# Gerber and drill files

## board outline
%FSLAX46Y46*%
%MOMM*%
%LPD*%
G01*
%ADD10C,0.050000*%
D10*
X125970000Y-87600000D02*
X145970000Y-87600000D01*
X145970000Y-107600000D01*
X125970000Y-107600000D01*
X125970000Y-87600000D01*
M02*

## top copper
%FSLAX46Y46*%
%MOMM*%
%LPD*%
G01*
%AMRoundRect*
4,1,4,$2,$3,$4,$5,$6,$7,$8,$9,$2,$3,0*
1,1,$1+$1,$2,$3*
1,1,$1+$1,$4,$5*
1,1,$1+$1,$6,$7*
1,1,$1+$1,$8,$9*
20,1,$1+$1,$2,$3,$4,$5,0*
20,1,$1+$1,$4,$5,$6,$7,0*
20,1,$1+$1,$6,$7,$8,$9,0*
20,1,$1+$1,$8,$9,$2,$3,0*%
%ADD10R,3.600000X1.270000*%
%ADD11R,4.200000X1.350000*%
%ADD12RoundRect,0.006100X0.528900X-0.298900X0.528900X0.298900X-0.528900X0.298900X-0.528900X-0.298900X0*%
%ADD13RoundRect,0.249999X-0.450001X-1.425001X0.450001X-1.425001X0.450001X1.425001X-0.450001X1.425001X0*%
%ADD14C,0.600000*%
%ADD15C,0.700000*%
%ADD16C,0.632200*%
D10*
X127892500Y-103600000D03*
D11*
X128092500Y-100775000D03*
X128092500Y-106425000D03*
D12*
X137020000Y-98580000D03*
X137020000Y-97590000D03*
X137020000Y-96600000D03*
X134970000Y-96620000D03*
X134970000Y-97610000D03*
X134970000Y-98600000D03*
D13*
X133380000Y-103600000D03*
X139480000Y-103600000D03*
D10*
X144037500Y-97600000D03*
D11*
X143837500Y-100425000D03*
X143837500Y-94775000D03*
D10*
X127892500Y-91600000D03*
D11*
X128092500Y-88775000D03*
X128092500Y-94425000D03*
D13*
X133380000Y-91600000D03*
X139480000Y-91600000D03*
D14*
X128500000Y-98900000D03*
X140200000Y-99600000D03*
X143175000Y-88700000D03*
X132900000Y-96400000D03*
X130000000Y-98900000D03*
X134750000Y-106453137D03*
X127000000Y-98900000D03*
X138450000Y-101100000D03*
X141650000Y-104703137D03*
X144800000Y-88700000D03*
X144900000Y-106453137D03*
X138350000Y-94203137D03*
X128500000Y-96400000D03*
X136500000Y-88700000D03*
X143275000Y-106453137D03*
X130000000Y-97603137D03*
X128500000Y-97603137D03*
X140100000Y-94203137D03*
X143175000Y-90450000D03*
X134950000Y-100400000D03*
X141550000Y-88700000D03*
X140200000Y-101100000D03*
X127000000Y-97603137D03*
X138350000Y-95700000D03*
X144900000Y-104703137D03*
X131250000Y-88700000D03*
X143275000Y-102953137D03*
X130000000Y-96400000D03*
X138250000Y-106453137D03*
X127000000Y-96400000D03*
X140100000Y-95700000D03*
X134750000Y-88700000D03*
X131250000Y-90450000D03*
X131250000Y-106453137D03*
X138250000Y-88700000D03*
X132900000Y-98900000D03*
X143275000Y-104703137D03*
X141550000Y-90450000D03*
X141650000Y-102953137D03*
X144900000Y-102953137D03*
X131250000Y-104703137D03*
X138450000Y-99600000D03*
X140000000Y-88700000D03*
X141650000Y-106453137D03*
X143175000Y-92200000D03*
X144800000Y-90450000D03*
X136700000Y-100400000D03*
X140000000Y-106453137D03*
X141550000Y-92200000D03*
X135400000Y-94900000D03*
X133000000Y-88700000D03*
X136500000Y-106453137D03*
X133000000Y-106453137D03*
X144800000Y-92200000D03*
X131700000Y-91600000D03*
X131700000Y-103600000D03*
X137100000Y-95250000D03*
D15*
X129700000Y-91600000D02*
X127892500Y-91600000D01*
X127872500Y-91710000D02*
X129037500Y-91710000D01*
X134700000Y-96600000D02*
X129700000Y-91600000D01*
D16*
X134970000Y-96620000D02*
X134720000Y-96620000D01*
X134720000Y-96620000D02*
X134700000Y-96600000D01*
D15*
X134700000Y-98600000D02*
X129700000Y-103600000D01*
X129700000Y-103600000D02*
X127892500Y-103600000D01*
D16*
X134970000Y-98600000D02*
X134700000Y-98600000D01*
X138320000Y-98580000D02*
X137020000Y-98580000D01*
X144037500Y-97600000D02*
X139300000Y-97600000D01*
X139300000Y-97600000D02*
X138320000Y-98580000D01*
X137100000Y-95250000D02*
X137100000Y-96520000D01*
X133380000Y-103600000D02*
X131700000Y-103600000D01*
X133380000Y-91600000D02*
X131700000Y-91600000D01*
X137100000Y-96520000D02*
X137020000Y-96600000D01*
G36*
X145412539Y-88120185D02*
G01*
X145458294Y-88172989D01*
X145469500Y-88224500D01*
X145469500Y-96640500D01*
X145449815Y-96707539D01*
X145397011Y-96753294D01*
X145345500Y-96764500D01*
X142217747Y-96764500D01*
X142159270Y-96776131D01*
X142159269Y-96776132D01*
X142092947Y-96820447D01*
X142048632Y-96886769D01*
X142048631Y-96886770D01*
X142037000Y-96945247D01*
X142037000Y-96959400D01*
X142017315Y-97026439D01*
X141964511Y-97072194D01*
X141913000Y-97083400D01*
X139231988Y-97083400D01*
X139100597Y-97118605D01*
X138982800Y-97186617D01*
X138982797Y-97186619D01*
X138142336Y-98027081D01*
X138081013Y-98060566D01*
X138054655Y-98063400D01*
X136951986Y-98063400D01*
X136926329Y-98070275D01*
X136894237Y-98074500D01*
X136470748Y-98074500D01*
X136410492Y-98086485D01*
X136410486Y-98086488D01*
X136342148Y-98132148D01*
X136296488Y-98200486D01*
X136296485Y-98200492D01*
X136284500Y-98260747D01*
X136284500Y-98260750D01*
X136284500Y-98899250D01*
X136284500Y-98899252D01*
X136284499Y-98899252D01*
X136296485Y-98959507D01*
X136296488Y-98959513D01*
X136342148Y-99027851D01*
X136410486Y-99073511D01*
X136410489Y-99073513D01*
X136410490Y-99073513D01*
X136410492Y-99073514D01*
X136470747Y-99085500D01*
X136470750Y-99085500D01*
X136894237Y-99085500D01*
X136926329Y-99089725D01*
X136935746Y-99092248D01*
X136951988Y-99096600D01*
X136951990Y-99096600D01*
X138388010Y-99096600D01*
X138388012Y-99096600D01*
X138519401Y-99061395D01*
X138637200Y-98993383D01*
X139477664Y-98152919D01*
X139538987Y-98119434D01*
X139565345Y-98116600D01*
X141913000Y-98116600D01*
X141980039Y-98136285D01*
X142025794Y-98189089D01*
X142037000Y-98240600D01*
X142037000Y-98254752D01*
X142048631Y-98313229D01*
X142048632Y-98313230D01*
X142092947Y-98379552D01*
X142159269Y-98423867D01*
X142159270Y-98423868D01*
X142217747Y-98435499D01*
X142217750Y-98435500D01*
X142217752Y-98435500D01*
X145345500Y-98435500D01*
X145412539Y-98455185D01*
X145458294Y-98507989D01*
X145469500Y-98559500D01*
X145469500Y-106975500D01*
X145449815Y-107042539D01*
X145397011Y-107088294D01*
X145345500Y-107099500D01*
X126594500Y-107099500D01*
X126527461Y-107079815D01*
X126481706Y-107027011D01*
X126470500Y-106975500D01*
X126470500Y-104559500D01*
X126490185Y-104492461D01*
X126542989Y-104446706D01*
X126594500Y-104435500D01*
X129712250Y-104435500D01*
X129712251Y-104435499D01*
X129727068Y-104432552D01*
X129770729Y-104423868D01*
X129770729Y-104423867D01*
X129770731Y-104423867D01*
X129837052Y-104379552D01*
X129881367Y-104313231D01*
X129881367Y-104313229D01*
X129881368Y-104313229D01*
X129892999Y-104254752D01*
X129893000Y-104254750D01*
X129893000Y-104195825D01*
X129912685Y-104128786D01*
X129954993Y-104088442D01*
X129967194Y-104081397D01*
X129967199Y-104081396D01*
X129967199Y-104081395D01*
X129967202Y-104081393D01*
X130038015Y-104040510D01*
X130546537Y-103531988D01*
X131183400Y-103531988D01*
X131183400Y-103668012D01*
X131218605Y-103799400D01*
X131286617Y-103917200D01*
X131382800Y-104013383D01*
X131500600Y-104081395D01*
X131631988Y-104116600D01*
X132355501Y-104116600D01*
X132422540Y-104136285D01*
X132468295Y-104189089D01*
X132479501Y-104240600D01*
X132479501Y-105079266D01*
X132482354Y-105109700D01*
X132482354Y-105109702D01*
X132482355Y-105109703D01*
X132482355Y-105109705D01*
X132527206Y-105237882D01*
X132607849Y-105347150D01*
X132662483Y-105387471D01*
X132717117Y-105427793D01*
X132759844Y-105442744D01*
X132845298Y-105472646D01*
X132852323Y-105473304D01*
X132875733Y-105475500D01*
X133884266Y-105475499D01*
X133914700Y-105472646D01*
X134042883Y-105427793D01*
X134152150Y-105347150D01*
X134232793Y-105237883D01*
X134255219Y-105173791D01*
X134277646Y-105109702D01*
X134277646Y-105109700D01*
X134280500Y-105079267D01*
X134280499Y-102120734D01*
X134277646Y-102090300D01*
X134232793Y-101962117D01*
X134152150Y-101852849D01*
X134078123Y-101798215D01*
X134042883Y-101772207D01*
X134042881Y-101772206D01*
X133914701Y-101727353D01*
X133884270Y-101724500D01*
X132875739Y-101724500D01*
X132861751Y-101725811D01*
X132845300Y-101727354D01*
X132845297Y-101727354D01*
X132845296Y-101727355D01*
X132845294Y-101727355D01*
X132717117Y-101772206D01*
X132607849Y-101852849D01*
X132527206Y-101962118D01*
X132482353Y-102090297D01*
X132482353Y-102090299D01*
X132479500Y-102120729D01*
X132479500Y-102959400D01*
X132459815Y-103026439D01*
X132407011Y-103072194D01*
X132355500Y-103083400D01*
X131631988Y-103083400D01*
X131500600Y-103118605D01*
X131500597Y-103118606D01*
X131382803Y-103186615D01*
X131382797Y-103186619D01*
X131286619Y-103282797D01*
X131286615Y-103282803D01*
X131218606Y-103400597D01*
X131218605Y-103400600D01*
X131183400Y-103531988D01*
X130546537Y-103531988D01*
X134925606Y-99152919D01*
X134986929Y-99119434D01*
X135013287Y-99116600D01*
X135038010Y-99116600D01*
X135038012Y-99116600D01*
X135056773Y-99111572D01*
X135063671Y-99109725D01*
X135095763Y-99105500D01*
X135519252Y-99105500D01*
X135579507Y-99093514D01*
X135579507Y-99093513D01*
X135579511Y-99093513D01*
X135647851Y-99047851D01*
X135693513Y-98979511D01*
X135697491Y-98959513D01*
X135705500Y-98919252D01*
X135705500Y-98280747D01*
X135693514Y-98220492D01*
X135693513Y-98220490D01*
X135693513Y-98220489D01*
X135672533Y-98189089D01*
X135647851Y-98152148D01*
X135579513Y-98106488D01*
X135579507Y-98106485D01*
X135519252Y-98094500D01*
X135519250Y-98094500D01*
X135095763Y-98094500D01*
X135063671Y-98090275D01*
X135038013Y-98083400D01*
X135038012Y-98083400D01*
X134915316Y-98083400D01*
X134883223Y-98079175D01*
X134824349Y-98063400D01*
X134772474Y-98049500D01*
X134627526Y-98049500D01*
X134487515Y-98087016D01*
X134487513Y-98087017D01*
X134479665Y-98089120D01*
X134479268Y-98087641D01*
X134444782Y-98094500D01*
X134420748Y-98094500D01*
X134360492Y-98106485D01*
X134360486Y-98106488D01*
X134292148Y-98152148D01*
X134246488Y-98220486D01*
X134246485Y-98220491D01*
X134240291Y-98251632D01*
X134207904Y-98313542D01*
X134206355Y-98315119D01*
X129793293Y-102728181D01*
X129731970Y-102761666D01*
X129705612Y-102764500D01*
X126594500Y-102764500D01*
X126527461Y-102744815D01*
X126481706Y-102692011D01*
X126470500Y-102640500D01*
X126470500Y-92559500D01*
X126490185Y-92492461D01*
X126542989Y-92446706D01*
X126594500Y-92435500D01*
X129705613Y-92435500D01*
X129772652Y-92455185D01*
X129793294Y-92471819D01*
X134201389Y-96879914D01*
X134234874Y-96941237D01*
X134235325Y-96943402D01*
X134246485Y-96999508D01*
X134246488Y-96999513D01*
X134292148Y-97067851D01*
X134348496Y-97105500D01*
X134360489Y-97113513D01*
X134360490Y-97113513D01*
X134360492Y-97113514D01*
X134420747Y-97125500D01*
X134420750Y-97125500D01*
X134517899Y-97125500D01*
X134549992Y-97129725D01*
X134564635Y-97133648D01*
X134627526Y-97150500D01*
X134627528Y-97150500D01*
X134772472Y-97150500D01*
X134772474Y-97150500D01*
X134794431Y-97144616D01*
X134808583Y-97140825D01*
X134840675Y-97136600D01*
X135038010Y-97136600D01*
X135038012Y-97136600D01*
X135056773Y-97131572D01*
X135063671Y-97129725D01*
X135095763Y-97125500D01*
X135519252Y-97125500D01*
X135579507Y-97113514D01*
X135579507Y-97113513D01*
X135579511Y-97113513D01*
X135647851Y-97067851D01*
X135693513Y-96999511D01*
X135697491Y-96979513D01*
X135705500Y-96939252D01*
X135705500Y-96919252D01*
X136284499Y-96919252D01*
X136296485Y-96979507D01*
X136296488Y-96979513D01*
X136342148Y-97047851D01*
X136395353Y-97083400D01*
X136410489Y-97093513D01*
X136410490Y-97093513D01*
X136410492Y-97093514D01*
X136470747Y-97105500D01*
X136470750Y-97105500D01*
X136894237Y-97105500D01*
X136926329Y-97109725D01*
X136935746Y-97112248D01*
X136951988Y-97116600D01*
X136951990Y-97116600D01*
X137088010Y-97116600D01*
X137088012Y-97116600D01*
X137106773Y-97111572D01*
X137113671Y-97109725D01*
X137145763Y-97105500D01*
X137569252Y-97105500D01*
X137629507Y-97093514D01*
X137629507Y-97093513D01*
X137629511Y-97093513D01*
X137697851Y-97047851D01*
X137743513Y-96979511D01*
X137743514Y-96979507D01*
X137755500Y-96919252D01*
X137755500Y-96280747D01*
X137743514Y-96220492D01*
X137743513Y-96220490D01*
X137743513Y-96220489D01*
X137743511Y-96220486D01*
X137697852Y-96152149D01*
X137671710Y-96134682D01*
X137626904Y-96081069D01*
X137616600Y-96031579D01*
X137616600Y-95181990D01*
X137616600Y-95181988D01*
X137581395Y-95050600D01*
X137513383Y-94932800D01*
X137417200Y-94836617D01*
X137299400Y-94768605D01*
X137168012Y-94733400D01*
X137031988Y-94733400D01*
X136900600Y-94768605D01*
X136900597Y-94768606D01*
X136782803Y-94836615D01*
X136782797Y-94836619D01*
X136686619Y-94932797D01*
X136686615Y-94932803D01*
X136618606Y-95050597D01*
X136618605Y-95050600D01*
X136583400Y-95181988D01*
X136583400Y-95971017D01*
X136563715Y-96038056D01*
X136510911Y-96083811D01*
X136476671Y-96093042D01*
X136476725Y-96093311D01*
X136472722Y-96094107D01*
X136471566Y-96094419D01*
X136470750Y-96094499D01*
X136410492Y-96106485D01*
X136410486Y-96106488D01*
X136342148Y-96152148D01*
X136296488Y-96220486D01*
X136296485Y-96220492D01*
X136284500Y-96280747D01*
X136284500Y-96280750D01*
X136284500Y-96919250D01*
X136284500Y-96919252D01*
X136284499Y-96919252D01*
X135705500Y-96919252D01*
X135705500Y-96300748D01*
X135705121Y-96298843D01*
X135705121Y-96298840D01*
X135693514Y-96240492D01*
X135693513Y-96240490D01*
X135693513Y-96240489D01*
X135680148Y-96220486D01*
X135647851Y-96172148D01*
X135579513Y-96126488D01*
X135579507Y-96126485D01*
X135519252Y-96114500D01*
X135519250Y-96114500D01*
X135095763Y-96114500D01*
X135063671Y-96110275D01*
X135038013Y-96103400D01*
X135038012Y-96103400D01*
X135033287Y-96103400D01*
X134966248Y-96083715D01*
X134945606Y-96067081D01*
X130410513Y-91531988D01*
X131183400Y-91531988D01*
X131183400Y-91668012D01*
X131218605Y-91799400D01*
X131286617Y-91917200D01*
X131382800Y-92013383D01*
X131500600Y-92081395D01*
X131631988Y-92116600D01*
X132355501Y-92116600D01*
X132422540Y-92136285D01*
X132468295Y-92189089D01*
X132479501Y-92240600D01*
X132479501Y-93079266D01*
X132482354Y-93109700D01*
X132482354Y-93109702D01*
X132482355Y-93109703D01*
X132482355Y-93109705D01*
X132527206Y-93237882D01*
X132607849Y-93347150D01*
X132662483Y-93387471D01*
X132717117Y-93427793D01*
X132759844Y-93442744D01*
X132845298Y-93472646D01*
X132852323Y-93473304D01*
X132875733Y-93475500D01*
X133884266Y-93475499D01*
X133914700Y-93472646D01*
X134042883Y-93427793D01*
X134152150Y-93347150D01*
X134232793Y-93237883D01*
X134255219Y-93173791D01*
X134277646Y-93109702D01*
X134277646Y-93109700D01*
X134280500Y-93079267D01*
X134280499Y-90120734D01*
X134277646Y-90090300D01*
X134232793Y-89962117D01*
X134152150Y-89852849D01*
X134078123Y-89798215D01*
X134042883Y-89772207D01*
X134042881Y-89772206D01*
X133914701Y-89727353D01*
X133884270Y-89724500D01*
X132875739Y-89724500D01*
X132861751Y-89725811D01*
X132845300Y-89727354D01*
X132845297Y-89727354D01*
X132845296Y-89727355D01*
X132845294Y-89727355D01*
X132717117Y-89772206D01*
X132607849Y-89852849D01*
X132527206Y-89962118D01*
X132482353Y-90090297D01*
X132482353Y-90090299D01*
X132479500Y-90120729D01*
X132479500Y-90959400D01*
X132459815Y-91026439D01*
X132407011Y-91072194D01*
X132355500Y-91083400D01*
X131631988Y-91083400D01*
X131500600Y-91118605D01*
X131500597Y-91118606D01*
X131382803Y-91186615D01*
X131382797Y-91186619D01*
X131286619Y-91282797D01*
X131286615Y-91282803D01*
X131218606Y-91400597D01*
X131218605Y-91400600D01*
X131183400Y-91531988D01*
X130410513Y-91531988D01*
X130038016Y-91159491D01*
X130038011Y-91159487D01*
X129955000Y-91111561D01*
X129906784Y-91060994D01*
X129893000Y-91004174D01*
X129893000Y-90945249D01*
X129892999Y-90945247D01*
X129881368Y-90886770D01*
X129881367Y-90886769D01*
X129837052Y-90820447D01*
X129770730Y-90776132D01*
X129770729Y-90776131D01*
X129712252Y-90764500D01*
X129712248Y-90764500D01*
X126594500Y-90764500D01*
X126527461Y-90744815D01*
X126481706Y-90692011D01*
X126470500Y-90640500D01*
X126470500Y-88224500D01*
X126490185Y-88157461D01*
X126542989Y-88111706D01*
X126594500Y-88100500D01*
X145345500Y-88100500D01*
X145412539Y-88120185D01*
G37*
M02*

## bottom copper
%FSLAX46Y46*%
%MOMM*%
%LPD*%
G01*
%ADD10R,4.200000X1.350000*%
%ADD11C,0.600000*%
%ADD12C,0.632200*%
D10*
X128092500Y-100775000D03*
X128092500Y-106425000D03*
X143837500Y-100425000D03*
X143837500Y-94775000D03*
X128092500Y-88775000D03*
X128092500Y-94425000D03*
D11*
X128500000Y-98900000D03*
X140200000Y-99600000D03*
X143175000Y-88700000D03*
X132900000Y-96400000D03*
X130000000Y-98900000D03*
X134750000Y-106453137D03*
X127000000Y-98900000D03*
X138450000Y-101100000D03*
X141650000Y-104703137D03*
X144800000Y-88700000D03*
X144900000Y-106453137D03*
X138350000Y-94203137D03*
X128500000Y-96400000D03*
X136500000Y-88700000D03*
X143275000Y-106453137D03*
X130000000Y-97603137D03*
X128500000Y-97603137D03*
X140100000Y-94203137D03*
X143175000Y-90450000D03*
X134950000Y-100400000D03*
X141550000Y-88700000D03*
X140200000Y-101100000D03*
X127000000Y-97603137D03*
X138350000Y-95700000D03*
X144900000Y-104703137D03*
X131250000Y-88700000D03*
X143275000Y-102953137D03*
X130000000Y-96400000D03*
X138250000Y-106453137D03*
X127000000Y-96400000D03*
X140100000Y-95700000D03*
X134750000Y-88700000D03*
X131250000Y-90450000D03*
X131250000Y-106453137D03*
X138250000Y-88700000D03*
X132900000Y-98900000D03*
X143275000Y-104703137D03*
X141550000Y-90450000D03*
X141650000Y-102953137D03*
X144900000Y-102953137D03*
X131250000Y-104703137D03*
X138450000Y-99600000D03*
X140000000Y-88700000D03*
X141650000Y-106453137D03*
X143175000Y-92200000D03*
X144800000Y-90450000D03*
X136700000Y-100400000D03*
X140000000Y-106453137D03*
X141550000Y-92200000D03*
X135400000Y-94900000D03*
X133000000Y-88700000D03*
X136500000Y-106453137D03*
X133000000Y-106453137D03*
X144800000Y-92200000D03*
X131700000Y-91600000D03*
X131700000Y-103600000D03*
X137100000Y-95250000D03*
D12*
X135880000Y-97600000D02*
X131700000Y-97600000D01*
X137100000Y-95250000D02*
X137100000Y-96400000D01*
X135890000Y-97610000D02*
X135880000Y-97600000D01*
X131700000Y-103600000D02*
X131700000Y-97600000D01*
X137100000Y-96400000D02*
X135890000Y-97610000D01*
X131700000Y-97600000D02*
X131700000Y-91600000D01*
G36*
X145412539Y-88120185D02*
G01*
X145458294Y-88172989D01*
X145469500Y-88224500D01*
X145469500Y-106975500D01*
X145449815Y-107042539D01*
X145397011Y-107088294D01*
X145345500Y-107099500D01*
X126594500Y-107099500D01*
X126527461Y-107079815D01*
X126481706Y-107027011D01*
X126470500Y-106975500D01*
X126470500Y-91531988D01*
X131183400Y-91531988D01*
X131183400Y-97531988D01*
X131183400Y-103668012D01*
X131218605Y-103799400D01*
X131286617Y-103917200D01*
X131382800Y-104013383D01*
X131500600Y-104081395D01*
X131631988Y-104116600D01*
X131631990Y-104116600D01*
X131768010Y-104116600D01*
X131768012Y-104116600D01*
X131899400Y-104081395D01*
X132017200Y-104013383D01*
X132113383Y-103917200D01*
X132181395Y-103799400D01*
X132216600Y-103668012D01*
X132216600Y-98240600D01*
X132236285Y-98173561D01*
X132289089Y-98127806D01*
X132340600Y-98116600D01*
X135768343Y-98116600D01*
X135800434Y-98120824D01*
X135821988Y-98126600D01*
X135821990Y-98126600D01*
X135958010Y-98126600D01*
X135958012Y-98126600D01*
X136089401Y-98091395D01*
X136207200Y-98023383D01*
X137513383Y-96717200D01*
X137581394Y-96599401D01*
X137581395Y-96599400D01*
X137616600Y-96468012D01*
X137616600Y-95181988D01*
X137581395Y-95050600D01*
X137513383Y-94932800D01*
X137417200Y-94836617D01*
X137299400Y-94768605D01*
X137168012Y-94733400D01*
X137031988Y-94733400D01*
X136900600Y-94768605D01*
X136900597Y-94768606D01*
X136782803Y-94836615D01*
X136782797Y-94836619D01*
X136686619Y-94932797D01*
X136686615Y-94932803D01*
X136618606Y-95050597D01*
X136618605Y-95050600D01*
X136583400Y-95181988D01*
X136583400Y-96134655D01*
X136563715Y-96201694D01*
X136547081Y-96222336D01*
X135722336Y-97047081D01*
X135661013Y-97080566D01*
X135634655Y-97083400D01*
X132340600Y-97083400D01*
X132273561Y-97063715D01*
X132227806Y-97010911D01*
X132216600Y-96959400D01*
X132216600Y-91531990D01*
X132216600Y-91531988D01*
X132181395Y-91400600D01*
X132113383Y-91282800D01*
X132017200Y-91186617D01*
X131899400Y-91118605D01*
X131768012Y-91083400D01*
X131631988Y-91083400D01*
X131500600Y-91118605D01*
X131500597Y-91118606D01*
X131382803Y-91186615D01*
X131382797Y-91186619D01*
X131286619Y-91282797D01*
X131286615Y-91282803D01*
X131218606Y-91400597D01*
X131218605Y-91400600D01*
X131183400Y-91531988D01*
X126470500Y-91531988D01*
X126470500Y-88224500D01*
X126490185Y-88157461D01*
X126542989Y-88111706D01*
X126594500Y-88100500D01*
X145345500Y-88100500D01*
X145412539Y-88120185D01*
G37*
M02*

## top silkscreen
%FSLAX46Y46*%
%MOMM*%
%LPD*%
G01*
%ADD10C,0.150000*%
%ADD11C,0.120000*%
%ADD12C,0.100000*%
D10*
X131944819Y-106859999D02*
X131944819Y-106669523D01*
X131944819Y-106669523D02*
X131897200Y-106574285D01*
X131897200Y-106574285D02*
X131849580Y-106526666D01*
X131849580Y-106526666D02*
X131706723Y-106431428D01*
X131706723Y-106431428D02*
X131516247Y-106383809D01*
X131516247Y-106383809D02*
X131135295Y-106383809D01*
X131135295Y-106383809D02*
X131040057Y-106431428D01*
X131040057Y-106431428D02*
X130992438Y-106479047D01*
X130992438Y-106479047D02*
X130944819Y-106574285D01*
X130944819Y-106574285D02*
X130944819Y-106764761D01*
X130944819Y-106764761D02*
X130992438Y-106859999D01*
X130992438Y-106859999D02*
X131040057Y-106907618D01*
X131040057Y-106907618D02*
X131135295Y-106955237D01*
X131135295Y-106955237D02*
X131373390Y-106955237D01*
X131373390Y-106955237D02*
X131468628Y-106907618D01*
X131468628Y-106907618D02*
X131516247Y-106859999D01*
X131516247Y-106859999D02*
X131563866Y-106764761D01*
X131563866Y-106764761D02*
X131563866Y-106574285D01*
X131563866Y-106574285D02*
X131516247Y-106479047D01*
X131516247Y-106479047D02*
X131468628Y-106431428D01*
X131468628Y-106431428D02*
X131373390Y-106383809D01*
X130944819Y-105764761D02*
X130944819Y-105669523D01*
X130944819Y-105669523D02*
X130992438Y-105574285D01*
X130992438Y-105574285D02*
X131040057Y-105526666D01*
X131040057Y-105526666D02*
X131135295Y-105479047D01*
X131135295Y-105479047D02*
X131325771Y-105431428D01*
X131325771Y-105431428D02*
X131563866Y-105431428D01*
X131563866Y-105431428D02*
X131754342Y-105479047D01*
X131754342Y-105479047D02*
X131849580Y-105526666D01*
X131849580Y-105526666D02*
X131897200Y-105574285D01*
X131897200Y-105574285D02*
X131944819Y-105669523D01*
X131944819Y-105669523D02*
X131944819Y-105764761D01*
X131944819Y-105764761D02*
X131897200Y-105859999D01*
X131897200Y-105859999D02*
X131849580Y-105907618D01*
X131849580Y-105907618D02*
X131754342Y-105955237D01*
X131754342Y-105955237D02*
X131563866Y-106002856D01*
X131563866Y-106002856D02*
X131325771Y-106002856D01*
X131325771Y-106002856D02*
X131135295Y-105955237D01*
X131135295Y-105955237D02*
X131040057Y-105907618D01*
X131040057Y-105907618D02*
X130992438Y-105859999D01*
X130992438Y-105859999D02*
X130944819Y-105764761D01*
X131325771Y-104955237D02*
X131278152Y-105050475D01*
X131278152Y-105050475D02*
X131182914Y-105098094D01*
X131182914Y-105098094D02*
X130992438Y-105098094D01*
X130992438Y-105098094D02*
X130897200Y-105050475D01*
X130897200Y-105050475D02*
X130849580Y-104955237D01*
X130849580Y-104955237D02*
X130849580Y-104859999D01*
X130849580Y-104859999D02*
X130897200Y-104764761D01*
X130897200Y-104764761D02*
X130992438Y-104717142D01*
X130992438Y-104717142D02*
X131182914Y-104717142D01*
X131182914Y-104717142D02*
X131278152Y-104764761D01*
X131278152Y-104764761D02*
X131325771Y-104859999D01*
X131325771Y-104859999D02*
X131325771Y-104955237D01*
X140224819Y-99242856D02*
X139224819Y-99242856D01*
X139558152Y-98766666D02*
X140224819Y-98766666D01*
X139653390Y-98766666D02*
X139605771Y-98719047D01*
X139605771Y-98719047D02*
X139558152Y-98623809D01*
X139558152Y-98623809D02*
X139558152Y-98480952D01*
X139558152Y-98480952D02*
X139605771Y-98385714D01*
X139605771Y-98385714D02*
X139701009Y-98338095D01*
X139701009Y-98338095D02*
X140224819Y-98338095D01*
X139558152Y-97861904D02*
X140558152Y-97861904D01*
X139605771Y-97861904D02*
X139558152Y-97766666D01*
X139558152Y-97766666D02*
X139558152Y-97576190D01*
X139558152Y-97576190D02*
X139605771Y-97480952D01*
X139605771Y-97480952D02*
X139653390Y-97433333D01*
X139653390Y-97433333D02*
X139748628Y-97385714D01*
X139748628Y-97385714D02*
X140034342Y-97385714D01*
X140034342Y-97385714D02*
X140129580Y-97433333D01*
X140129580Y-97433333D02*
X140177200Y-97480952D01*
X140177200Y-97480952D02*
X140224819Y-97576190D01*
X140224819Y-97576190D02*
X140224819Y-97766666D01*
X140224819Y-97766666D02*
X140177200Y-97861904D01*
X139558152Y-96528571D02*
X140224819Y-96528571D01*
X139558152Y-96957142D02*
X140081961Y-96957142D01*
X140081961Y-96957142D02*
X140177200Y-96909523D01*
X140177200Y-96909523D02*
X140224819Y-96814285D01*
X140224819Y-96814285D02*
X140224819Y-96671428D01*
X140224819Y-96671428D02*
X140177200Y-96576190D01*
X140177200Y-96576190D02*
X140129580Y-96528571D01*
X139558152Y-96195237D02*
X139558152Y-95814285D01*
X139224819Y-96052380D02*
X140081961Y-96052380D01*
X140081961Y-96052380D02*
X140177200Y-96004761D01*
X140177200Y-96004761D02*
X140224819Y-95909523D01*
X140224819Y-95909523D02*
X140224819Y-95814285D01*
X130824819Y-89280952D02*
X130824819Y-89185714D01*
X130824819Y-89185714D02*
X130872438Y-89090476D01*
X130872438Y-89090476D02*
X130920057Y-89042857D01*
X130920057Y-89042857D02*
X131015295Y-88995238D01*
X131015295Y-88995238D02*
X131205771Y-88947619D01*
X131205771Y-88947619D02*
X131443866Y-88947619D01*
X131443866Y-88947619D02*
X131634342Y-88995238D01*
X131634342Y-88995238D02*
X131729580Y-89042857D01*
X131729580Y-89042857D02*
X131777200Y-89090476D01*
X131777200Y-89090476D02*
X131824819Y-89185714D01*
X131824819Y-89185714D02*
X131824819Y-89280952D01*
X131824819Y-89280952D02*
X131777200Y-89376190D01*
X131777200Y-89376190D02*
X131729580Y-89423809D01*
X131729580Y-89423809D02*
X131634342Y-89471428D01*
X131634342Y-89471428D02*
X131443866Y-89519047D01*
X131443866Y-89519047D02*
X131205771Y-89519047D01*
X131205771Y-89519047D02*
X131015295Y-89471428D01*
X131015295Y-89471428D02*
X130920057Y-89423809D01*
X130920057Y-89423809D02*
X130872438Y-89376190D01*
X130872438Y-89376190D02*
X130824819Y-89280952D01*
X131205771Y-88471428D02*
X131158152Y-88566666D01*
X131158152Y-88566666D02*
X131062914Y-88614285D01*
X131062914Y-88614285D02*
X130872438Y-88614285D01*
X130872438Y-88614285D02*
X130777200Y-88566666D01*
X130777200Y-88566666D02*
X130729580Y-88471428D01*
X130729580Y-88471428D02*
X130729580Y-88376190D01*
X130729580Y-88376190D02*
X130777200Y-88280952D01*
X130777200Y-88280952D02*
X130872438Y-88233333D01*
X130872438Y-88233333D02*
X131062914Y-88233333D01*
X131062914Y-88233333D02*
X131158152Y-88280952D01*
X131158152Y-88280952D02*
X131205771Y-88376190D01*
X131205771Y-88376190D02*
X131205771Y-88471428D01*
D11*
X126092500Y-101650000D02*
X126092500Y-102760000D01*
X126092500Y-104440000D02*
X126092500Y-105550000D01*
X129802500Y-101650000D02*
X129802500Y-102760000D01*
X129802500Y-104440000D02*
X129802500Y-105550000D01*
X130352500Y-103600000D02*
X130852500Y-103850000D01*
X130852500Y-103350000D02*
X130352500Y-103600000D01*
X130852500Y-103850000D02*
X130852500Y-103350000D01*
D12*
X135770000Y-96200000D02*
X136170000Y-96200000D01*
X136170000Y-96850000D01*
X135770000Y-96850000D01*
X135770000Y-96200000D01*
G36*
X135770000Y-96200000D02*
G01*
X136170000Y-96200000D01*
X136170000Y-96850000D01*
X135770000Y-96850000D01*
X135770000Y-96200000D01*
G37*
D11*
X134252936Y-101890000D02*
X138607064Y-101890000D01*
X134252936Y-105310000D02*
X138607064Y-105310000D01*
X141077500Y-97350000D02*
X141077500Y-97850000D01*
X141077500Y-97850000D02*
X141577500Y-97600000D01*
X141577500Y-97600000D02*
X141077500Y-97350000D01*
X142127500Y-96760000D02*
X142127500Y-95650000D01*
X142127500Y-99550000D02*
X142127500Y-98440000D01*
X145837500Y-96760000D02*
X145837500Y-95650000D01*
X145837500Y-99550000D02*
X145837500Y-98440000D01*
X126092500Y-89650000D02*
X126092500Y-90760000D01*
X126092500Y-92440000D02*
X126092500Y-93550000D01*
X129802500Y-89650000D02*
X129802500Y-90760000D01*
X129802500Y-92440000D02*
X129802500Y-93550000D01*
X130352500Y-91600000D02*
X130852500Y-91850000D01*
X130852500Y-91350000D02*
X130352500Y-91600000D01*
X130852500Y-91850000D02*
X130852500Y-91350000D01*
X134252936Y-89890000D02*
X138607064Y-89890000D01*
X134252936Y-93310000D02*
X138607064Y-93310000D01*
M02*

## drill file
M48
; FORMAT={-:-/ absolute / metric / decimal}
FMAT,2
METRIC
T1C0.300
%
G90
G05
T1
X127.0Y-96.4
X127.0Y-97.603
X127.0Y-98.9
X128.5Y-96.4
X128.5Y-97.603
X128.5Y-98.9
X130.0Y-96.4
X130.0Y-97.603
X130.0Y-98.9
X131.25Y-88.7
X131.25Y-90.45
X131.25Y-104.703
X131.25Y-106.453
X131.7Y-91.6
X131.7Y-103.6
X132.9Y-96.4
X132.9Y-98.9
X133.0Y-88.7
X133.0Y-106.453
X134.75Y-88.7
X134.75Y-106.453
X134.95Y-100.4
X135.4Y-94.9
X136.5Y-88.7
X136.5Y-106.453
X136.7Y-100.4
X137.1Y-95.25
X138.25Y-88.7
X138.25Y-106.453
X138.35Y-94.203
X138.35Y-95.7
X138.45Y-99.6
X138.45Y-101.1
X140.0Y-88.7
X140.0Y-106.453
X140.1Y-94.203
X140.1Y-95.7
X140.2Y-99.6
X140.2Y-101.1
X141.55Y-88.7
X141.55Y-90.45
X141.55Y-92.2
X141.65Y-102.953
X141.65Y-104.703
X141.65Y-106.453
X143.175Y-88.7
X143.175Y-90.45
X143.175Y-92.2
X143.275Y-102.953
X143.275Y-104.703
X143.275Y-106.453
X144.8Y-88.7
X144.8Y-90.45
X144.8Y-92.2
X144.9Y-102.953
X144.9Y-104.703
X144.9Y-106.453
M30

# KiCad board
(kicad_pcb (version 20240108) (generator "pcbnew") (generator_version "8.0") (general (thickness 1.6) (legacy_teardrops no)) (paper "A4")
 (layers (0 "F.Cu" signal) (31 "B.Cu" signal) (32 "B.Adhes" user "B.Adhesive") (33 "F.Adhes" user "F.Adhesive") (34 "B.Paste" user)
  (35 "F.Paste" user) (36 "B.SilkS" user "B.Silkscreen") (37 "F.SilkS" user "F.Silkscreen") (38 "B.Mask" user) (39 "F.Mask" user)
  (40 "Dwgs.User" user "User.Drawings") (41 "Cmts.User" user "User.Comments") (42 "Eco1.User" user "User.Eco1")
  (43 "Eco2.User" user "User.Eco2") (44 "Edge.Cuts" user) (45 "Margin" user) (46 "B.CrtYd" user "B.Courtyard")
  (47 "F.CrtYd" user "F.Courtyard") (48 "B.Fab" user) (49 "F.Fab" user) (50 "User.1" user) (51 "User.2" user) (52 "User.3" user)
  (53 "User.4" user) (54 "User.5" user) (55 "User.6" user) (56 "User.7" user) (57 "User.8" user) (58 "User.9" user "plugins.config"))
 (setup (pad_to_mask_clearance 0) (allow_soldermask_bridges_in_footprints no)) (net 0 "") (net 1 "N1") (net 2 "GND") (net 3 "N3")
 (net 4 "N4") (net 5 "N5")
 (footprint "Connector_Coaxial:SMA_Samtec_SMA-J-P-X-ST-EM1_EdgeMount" (layer "F.Cu") (at 128.0925 103.6 -90)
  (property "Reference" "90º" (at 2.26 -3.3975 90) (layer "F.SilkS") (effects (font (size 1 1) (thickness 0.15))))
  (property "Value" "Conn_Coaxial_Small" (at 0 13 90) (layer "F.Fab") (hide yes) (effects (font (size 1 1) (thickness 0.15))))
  (fp_line (start -1.95 2) (end -0.84 2) (stroke (width 0.12) (type solid)) (layer "F.SilkS"))
  (fp_line (start 0.84 2) (end 1.95 2) (stroke (width 0.12) (type solid)) (layer "F.SilkS"))
  (fp_line (start -1.95 -1.71) (end -0.84 -1.71) (stroke (width 0.12) (type solid)) (layer "F.SilkS"))
  (fp_line (start 0.84 -1.71) (end 1.95 -1.71) (stroke (width 0.12) (type solid)) (layer "F.SilkS"))
  (fp_line (start 0 -2.26) (end 0.25 -2.76) (stroke (width 0.12) (type solid)) (layer "F.SilkS"))
  (fp_line (start -0.25 -2.76) (end 0 -2.26) (stroke (width 0.12) (type solid)) (layer "F.SilkS"))
  (fp_line (start 0.25 -2.76) (end -0.25 -2.76) (stroke (width 0.12) (type solid)) (layer "F.SilkS"))
  (pad "1" smd rect (at 0 0.2 270) (size 1.27 3.6) (layers "F.Cu" "F.Paste" "F.Mask") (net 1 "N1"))
  (pad "2" smd rect (at -2.825 0 270) (size 1.35 4.2) (layers "F.Cu" "F.Paste" "F.Mask") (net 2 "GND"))
  (pad "2" smd rect (at -2.825 0 270) (size 1.35 4.2) (layers "B.Cu" "B.Paste" "B.Mask") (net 2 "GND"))
  (pad "2" smd rect (at 2.825 0 270) (size 1.35 4.2) (layers "F.Cu" "F.Paste" "F.Mask") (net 2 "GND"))
  (pad "2" smd rect (at 2.825 0 270) (size 1.35 4.2) (layers "B.Cu" "B.Paste" "B.Mask") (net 2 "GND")))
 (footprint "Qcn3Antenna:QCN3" (layer "F.Cu") (at 136.97 97.6 90)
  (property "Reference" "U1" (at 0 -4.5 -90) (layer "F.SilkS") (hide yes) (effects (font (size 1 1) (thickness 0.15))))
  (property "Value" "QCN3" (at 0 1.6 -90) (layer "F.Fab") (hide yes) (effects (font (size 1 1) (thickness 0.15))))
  (fp_rect (start 0.75 -1.2) (end 1.4 -0.8) (stroke (width 0.1) (type solid)) (fill solid) (layer "F.SilkS"))
  (pad "1" smd roundrect (at -0.98 0.05 90) (size 0.61 1.07) (layers "F.Cu" "F.Paste" "F.Mask") (roundrect_rratio 0.01) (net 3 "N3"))
  (pad "2" smd roundrect (at 0.01 0.05 90) (size 0.61 1.07) (layers "F.Cu" "F.Paste" "F.Mask") (roundrect_rratio 0.01) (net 2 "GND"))
  (pad "3" smd roundrect (at 1 0.05 90) (size 0.61 1.07) (layers "F.Cu" "F.Paste" "F.Mask") (roundrect_rratio 0.01) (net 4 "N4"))
  (pad "4" smd roundrect (at 0.98 -2 90) (size 0.61 1.07) (layers "F.Cu" "F.Paste" "F.Mask") (roundrect_rratio 0.01) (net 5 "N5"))
  (pad "5" smd roundrect (at -0.01 -2 90) (size 0.61 1.07) (layers "F.Cu" "F.Paste" "F.Mask") (roundrect_rratio 0.01) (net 2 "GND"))
  (pad "6" smd roundrect (at -1 -2 90) (size 0.61 1.07) (layers "F.Cu" "F.Paste" "F.Mask") (roundrect_rratio 0.01) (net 1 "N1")))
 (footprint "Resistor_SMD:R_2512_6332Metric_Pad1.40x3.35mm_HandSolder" (layer "F.Cu") (at 136.43 103.6)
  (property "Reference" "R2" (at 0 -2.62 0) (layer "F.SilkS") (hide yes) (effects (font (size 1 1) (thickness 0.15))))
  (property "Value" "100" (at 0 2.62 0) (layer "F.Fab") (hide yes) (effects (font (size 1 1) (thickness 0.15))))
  (fp_line (start -2.177064 -1.71) (end 2.177064 -1.71) (stroke (width 0.12) (type solid)) (layer "F.SilkS"))
  (fp_line (start -2.177064 1.71) (end 2.177064 1.71) (stroke (width 0.12) (type solid)) (layer "F.SilkS"))
  (pad "1" smd roundrect (at -3.05 0) (size 1.4 3.35) (layers "F.Cu" "F.Paste" "F.Mask") (roundrect_rratio 0.178571) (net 4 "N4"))
  (pad "2" smd roundrect (at 3.05 0) (size 1.4 3.35) (layers "F.Cu" "F.Paste" "F.Mask") (roundrect_rratio 0.178571) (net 2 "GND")))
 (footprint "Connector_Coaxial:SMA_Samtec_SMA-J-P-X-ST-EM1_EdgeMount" (layer "F.Cu") (at 143.8375 97.6 90)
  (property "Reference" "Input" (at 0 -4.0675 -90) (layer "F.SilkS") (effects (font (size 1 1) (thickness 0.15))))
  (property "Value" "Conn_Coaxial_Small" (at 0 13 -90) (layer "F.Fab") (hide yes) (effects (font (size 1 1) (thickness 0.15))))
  (fp_line (start 0.25 -2.76) (end -0.25 -2.76) (stroke (width 0.12) (type solid)) (layer "F.SilkS"))
  (fp_line (start -0.25 -2.76) (end 0 -2.26) (stroke (width 0.12) (type solid)) (layer "F.SilkS"))
  (fp_line (start 0 -2.26) (end 0.25 -2.76) (stroke (width 0.12) (type solid)) (layer "F.SilkS"))
  (fp_line (start 0.84 -1.71) (end 1.95 -1.71) (stroke (width 0.12) (type solid)) (layer "F.SilkS"))
  (fp_line (start -1.95 -1.71) (end -0.84 -1.71) (stroke (width 0.12) (type solid)) (layer "F.SilkS"))
  (fp_line (start 0.84 2) (end 1.95 2) (stroke (width 0.12) (type solid)) (layer "F.SilkS"))
  (fp_line (start -1.95 2) (end -0.84 2) (stroke (width 0.12) (type solid)) (layer "F.SilkS"))
  (pad "1" smd rect (at 0 0.2 90) (size 1.27 3.6) (layers "F.Cu" "F.Paste" "F.Mask") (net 3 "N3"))
  (pad "2" smd rect (at -2.825 0 90) (size 1.35 4.2) (layers "F.Cu" "F.Paste" "F.Mask") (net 2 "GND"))
  (pad "2" smd rect (at -2.825 0 90) (size 1.35 4.2) (layers "B.Cu" "B.Paste" "B.Mask") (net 2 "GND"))
  (pad "2" smd rect (at 2.825 0 90) (size 1.35 4.2) (layers "F.Cu" "F.Paste" "F.Mask") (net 2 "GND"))
  (pad "2" smd rect (at 2.825 0 90) (size 1.35 4.2) (layers "B.Cu" "B.Paste" "B.Mask") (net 2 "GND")))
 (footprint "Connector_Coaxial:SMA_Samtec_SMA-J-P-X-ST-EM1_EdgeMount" (layer "F.Cu") (at 128.0925 91.6 -90)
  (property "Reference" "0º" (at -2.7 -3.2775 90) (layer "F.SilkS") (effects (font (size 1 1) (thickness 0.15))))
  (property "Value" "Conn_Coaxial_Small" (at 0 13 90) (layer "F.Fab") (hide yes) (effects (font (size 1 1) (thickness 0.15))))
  (fp_line (start -1.95 2) (end -0.84 2) (stroke (width 0.12) (type solid)) (layer "F.SilkS"))
  (fp_line (start 0.84 2) (end 1.95 2) (stroke (width 0.12) (type solid)) (layer "F.SilkS"))
  (fp_line (start -1.95 -1.71) (end -0.84 -1.71) (stroke (width 0.12) (type solid)) (layer "F.SilkS"))
  (fp_line (start 0.84 -1.71) (end 1.95 -1.71) (stroke (width 0.12) (type solid)) (layer "F.SilkS"))
  (fp_line (start 0 -2.26) (end 0.25 -2.76) (stroke (width 0.12) (type solid)) (layer "F.SilkS"))
  (fp_line (start -0.25 -2.76) (end 0 -2.26) (stroke (width 0.12) (type solid)) (layer "F.SilkS"))
  (fp_line (start 0.25 -2.76) (end -0.25 -2.76) (stroke (width 0.12) (type solid)) (layer "F.SilkS"))
  (pad "1" smd rect (at 0 0.2 270) (size 1.27 3.6) (layers "F.Cu" "F.Paste" "F.Mask") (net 5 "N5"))
  (pad "2" smd rect (at -2.825 0 270) (size 1.35 4.2) (layers "F.Cu" "F.Paste" "F.Mask") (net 2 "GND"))
  (pad "2" smd rect (at -2.825 0 270) (size 1.35 4.2) (layers "B.Cu" "B.Paste" "B.Mask") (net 2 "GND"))
  (pad "2" smd rect (at 2.825 0 270) (size 1.35 4.2) (layers "F.Cu" "F.Paste" "F.Mask") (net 2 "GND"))
  (pad "2" smd rect (at 2.825 0 270) (size 1.35 4.2) (layers "B.Cu" "B.Paste" "B.Mask") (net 2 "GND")))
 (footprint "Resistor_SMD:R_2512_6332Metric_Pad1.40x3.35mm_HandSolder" (layer "F.Cu") (at 136.43 91.6)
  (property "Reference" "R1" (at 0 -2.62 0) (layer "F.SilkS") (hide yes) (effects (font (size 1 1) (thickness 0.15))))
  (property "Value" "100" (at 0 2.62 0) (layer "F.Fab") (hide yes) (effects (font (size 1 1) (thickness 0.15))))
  (fp_line (start -2.177064 -1.71) (end 2.177064 -1.71) (stroke (width 0.12) (type solid)) (layer "F.SilkS"))
  (fp_line (start -2.177064 1.71) (end 2.177064 1.71) (stroke (width 0.12) (type solid)) (layer "F.SilkS"))
  (pad "1" smd roundrect (at -3.05 0) (size 1.4 3.35) (layers "F.Cu" "F.Paste" "F.Mask") (roundrect_rratio 0.178571) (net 4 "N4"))
  (pad "2" smd roundrect (at 3.05 0) (size 1.4 3.35) (layers "F.Cu" "F.Paste" "F.Mask") (roundrect_rratio 0.178571) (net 2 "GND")))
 (gr_rect (start 125.97 87.6) (end 145.97 107.6) (stroke (width 0.05) (type default)) (fill none) (layer "Edge.Cuts"))
 (via (at 128.5 98.9) (size 0.6) (drill 0.3) (layers "F.Cu" "B.Cu") (free yes) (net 2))
 (via (at 140.2 99.6) (size 0.6) (drill 0.3) (layers "F.Cu" "B.Cu") (free yes) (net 2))
 (via (at 143.175 88.7) (size 0.6) (drill 0.3) (layers "F.Cu" "B.Cu") (free yes) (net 2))
 (via (at 132.9 96.4) (size 0.6) (drill 0.3) (layers "F.Cu" "B.Cu") (free yes) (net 2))
 (via (at 130 98.9) (size 0.6) (drill 0.3) (layers "F.Cu" "B.Cu") (free yes) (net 2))
 (via (at 134.75 106.453137) (size 0.6) (drill 0.3) (layers "F.Cu" "B.Cu") (free yes) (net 2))
 (via (at 127 98.9) (size 0.6) (drill 0.3) (layers "F.Cu" "B.Cu") (free yes) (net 2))
 (via (at 138.45 101.1) (size 0.6) (drill 0.3) (layers "F.Cu" "B.Cu") (free yes) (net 2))
 (via (at 141.65 104.703137) (size 0.6) (drill 0.3) (layers "F.Cu" "B.Cu") (free yes) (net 2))
 (via (at 144.8 88.7) (size 0.6) (drill 0.3) (layers "F.Cu" "B.Cu") (free yes) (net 2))
 (via (at 144.9 106.453137) (size 0.6) (drill 0.3) (layers "F.Cu" "B.Cu") (free yes) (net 2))
 (via (at 138.35 94.203137) (size 0.6) (drill 0.3) (layers "F.Cu" "B.Cu") (free yes) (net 2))
 (via (at 128.5 96.4) (size 0.6) (drill 0.3) (layers "F.Cu" "B.Cu") (free yes) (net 2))
 (via (at 136.5 88.7) (size 0.6) (drill 0.3) (layers "F.Cu" "B.Cu") (free yes) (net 2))
 (via (at 143.275 106.453137) (size 0.6) (drill 0.3) (layers "F.Cu" "B.Cu") (free yes) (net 2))
 (via (at 130 97.603137) (size 0.6) (drill 0.3) (layers "F.Cu" "B.Cu") (free yes) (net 2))
 (via (at 128.5 97.603137) (size 0.6) (drill 0.3) (layers "F.Cu" "B.Cu") (free yes) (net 2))
 (via (at 140.1 94.203137) (size 0.6) (drill 0.3) (layers "F.Cu" "B.Cu") (free yes) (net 2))
 (via (at 143.175 90.45) (size 0.6) (drill 0.3) (layers "F.Cu" "B.Cu") (free yes) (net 2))
 (via (at 134.95 100.4) (size 0.6) (drill 0.3) (layers "F.Cu" "B.Cu") (free yes) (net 2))
 (via (at 141.55 88.7) (size 0.6) (drill 0.3) (layers "F.Cu" "B.Cu") (free yes) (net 2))
 (via (at 140.2 101.1) (size 0.6) (drill 0.3) (layers "F.Cu" "B.Cu") (free yes) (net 2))
 (via (at 127 97.603137) (size 0.6) (drill 0.3) (layers "F.Cu" "B.Cu") (free yes) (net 2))
 (via (at 138.35 95.7) (size 0.6) (drill 0.3) (layers "F.Cu" "B.Cu") (free yes) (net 2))
 (via (at 144.9 104.703137) (size 0.6) (drill 0.3) (layers "F.Cu" "B.Cu") (free yes) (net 2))
 (via (at 131.25 88.7) (size 0.6) (drill 0.3) (layers "F.Cu" "B.Cu") (free yes) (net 2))
 (via (at 143.275 102.953137) (size 0.6) (drill 0.3) (layers "F.Cu" "B.Cu") (free yes) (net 2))
 (via (at 130 96.4) (size 0.6) (drill 0.3) (layers "F.Cu" "B.Cu") (free yes) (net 2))
 (via (at 138.25 106.453137) (size 0.6) (drill 0.3) (layers "F.Cu" "B.Cu") (free yes) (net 2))
 (via (at 127 96.4) (size 0.6) (drill 0.3) (layers "F.Cu" "B.Cu") (free yes) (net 2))
 (via (at 140.1 95.7) (size 0.6) (drill 0.3) (layers "F.Cu" "B.Cu") (free yes) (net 2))
 (via (at 134.75 88.7) (size 0.6) (drill 0.3) (layers "F.Cu" "B.Cu") (free yes) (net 2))
 (via (at 131.25 90.45) (size 0.6) (drill 0.3) (layers "F.Cu" "B.Cu") (free yes) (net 2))
 (via (at 131.25 106.453137) (size 0.6) (drill 0.3) (layers "F.Cu" "B.Cu") (free yes) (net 2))
 (via (at 138.25 88.7) (size 0.6) (drill 0.3) (layers "F.Cu" "B.Cu") (free yes) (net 2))
 (via (at 132.9 98.9) (size 0.6) (drill 0.3) (layers "F.Cu" "B.Cu") (free yes) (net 2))
 (via (at 143.275 104.703137) (size 0.6) (drill 0.3) (layers "F.Cu" "B.Cu") (free yes) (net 2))
 (via (at 141.55 90.45) (size 0.6) (drill 0.3) (layers "F.Cu" "B.Cu") (free yes) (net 2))
 (via (at 141.65 102.953137) (size 0.6) (drill 0.3) (layers "F.Cu" "B.Cu") (free yes) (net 2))
 (via (at 144.9 102.953137) (size 0.6) (drill 0.3) (layers "F.Cu" "B.Cu") (free yes) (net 2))
 (via (at 131.25 104.703137) (size 0.6) (drill 0.3) (layers "F.Cu" "B.Cu") (free yes) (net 2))
 (via (at 138.45 99.6) (size 0.6) (drill 0.3) (layers "F.Cu" "B.Cu") (free yes) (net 2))
 (via (at 140 88.7) (size 0.6) (drill 0.3) (layers "F.Cu" "B.Cu") (free yes) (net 2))
 (via (at 141.65 106.453137) (size 0.6) (drill 0.3) (layers "F.Cu" "B.Cu") (free yes) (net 2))
 (via (at 143.175 92.2) (size 0.6) (drill 0.3) (layers "F.Cu" "B.Cu") (free yes) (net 2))
 (via (at 144.8 90.45) (size 0.6) (drill 0.3) (layers "F.Cu" "B.Cu") (free yes) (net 2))
 (via (at 136.7 100.4) (size 0.6) (drill 0.3) (layers "F.Cu" "B.Cu") (free yes) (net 2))
 (via (at 140 106.453137) (size 0.6) (drill 0.3) (layers "F.Cu" "B.Cu") (free yes) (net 2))
 (via (at 141.55 92.2) (size 0.6) (drill 0.3) (layers "F.Cu" "B.Cu") (free yes) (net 2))
 (via (at 135.4 94.9) (size 0.6) (drill 0.3) (layers "F.Cu" "B.Cu") (free yes) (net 2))
 (via (at 133 88.7) (size 0.6) (drill 0.3) (layers "F.Cu" "B.Cu") (free yes) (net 2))
 (via (at 136.5 106.453137) (size 0.6) (drill 0.3) (layers "F.Cu" "B.Cu") (free yes) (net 2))
 (via (at 133 106.453137) (size 0.6) (drill 0.3) (layers "F.Cu" "B.Cu") (free yes) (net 2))
 (via (at 144.8 92.2) (size 0.6) (drill 0.3) (layers "F.Cu" "B.Cu") (free yes) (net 2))
 (segment (start 129.7 91.6) (end 127.8925 91.6) (width 0.7) (layer "F.Cu") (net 5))
 (segment (start 127.8725 91.71) (end 129.0375 91.71) (width 0.7) (layer "F.Cu") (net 5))
 (segment (start 134.7 96.6) (end 129.7 91.6) (width 0.7) (layer "F.Cu") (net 5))
 (segment (start 134.97 96.62) (end 134.72 96.62) (width 0.6322) (layer "F.Cu") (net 5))
 (segment (start 134.72 96.62) (end 134.7 96.6) (width 0.6322) (layer "F.Cu") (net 5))
 (segment (start 134.7 98.6) (end 129.7 103.6) (width 0.7) (layer "F.Cu") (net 1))
 (segment (start 129.7 103.6) (end 127.8925 103.6) (width 0.7) (layer "F.Cu") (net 1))
 (segment (start 134.97 98.6) (end 134.7 98.6) (width 0.6322) (layer "F.Cu") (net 1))
 (segment (start 138.32 98.58) (end 137.02 98.58) (width 0.6322) (layer "F.Cu") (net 3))
 (segment (start 144.0375 97.6) (end 139.3 97.6) (width 0.6322) (layer "F.Cu") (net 3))
 (segment (start 139.3 97.6) (end 138.32 98.58) (width 0.6322) (layer "F.Cu") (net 3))
 (segment (start 137.1 95.25) (end 137.1 96.52) (width 0.6322) (layer "F.Cu") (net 4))
 (segment (start 133.38 103.6) (end 131.7 103.6) (width 0.6322) (layer "F.Cu") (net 4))
 (segment (start 133.38 91.6) (end 131.7 91.6) (width 0.6322) (layer "F.Cu") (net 4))
 (segment (start 137.1 96.52) (end 137.02 96.6) (width 0.6322) (layer "F.Cu") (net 4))
 (via (at 131.7 91.6) (size 0.6) (drill 0.3) (layers "F.Cu" "B.Cu") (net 4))
 (via (at 131.7 103.6) (size 0.6) (drill 0.3) (layers "F.Cu" "B.Cu") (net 4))
 (via (at 137.1 95.25) (size 0.6) (drill 0.3) (layers "F.Cu" "B.Cu") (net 4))
 (segment (start 135.88 97.6) (end 131.7 97.6) (width 0.6322) (layer "B.Cu") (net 4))
 (segment (start 137.1 95.25) (end 137.1 96.4) (width 0.6322) (layer "B.Cu") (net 4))
 (segment (start 135.89 97.61) (end 135.88 97.6) (width 0.6322) (layer "B.Cu") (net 4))
 (segment (start 131.7 103.6) (end 131.7 97.6) (width 0.6322) (layer "B.Cu") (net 4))
 (segment (start 137.1 96.4) (end 135.89 97.61) (width 0.6322) (layer "B.Cu") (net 4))
 (segment (start 131.7 97.6) (end 131.7 91.6) (width 0.6322) (layer "B.Cu") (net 4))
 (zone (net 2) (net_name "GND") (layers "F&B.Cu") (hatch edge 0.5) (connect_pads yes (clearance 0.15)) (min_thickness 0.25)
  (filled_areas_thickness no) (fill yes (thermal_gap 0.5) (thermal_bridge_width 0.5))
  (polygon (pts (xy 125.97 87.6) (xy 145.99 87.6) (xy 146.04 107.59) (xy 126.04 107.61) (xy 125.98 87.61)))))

